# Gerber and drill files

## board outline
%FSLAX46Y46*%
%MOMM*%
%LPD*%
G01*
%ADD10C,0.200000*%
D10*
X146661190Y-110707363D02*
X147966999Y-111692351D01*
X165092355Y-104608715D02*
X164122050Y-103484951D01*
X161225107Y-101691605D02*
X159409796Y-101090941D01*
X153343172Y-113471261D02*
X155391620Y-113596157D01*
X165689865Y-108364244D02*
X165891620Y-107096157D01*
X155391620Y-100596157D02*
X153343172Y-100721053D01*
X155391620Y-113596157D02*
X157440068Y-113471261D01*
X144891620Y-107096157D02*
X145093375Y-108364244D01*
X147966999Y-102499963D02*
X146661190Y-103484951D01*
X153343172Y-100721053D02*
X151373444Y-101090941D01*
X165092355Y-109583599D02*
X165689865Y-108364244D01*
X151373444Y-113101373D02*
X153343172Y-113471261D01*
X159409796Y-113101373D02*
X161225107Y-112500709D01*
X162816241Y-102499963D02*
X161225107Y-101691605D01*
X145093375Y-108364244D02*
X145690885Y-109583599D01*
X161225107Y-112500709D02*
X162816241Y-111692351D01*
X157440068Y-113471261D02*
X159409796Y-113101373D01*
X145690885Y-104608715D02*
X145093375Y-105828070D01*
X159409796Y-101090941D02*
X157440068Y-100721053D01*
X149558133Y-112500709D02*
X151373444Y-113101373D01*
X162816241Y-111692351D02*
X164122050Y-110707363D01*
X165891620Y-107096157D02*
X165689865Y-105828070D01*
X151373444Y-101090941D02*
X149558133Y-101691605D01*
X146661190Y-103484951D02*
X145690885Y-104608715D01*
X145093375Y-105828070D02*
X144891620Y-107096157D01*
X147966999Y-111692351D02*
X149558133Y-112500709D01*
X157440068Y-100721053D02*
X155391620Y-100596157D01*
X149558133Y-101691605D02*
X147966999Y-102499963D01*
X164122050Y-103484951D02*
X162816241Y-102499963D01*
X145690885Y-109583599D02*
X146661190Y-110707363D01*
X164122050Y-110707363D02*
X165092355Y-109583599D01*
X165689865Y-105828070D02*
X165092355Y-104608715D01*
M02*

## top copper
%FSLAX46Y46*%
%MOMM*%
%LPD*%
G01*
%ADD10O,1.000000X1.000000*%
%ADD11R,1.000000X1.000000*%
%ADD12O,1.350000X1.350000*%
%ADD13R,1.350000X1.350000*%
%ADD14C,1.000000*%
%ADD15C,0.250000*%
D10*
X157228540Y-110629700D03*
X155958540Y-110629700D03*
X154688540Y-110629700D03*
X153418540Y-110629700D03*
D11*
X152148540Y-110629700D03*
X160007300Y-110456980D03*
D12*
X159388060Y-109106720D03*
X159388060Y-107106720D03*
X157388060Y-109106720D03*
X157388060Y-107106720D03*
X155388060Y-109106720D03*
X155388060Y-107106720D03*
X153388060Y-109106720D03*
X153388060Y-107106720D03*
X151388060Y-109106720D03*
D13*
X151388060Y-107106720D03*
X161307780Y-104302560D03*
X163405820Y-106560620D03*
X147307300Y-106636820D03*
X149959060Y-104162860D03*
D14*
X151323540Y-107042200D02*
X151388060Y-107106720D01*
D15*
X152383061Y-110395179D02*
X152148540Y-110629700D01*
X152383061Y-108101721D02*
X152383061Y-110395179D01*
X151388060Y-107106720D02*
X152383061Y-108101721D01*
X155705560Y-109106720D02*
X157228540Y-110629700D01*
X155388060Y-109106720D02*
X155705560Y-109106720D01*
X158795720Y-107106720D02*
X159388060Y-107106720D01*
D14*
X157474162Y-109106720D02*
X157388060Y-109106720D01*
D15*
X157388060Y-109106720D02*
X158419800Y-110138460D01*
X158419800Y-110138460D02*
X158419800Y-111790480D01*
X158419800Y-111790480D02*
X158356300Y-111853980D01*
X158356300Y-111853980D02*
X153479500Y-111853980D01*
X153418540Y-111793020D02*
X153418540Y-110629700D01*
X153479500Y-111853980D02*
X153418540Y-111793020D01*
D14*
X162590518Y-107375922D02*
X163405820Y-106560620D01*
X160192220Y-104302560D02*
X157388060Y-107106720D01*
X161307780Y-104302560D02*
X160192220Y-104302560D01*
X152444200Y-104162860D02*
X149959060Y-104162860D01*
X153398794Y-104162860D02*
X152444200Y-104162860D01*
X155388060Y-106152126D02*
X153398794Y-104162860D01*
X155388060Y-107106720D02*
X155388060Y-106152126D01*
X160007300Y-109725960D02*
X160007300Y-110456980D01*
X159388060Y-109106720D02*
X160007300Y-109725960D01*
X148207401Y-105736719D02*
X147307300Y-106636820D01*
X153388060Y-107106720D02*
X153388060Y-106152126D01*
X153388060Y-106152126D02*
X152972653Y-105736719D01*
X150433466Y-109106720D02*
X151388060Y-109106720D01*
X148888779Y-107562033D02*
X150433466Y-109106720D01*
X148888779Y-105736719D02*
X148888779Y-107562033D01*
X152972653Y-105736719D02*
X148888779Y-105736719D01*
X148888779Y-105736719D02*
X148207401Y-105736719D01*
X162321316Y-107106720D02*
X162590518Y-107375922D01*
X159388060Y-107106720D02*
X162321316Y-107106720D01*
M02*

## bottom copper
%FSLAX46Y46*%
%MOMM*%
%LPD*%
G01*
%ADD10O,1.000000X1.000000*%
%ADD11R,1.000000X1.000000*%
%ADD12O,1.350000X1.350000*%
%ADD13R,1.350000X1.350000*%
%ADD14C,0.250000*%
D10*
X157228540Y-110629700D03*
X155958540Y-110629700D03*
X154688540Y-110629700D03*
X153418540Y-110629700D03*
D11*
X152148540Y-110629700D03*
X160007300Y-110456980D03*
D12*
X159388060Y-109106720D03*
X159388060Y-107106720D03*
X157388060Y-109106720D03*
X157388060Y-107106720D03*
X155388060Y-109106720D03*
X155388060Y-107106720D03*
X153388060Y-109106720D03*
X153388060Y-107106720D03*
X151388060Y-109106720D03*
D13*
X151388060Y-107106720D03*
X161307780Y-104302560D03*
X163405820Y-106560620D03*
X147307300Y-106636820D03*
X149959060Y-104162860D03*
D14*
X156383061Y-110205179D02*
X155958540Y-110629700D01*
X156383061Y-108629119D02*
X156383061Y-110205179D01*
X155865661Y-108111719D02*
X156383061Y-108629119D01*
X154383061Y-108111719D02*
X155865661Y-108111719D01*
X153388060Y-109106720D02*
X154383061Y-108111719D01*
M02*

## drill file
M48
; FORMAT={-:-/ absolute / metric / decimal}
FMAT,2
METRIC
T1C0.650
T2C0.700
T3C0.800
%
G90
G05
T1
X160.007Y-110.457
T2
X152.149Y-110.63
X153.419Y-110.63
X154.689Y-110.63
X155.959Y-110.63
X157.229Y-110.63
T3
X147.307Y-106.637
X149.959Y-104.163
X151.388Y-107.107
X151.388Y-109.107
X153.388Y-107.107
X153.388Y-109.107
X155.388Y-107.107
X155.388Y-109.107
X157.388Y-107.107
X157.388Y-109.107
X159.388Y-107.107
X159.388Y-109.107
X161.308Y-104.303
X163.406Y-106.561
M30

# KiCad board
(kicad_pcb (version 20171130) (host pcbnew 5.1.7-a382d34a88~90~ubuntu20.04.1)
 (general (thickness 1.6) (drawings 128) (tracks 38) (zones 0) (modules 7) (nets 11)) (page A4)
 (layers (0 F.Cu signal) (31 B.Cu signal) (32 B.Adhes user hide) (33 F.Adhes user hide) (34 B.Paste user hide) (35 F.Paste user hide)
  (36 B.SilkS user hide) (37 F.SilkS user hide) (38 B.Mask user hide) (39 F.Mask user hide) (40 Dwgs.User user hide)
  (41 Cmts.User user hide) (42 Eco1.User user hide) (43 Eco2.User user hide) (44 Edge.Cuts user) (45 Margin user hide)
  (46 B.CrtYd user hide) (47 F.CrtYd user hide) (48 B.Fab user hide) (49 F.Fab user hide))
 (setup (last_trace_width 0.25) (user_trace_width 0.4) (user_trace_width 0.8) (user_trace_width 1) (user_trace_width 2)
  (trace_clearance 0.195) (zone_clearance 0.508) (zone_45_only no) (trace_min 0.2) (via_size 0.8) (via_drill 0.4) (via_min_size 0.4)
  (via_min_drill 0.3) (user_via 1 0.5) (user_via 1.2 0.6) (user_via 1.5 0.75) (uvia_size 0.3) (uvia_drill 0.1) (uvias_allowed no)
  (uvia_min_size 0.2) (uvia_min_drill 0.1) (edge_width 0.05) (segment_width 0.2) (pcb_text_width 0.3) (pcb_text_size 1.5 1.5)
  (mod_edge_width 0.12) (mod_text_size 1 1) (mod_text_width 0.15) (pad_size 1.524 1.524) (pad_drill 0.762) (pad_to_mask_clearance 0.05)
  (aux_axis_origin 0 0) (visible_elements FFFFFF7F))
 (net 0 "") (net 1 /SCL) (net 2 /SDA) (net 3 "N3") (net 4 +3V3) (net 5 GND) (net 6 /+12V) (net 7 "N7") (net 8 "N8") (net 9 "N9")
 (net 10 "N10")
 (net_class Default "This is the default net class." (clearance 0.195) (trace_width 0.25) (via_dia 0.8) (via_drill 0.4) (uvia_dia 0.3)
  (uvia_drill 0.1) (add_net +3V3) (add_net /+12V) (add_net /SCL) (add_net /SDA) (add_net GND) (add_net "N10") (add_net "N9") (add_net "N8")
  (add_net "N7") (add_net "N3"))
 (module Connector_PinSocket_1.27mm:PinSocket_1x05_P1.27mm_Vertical (layer F.Cu) (at 152.14854 110.6297 90)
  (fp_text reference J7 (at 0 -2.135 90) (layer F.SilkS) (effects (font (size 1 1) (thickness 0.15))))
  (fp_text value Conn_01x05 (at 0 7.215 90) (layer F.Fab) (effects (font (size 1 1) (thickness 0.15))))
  (pad 5 thru_hole oval (at 0 5.08 90) (size 1 1) (drill 0.7) (layers *.Cu *.Mask) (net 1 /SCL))
  (pad 4 thru_hole oval (at 0 3.81 90) (size 1 1) (drill 0.7) (layers *.Cu *.Mask) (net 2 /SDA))
  (pad 3 thru_hole oval (at 0 2.54 90) (size 1 1) (drill 0.7) (layers *.Cu *.Mask) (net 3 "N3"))
  (pad 2 thru_hole oval (at 0 1.27 90) (size 1 1) (drill 0.7) (layers *.Cu *.Mask) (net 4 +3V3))
  (pad 1 thru_hole rect (at 0 0 90) (size 1 1) (drill 0.7) (layers *.Cu *.Mask) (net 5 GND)))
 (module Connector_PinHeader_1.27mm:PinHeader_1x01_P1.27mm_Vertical (layer F.Cu) (at 160.0073 110.45698)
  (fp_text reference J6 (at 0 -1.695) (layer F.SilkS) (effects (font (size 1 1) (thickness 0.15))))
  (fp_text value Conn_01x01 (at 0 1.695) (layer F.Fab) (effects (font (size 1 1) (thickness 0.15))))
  (pad 1 thru_hole rect (at 0 0) (size 1 1) (drill 0.65) (layers *.Cu *.Mask) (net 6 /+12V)))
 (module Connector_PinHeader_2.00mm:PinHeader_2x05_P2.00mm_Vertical (layer B.Cu) (at 151.38806 107.10672 270)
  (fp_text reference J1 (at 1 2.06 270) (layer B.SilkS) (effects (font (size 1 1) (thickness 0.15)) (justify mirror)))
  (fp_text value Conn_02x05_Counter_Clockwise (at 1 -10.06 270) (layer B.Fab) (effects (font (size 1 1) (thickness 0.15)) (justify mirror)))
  (pad 10 thru_hole oval (at 2 -8 270) (size 1.35 1.35) (drill 0.8) (layers *.Cu *.Mask) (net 6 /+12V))
  (pad 9 thru_hole oval (at 0 -8 270) (size 1.35 1.35) (drill 0.8) (layers *.Cu *.Mask) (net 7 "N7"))
  (pad 8 thru_hole oval (at 2 -6 270) (size 1.35 1.35) (drill 0.8) (layers *.Cu *.Mask) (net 4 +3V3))
  (pad 7 thru_hole oval (at 0 -6 270) (size 1.35 1.35) (drill 0.8) (layers *.Cu *.Mask) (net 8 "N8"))
  (pad 6 thru_hole oval (at 2 -4 270) (size 1.35 1.35) (drill 0.8) (layers *.Cu *.Mask) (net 1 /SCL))
  (pad 5 thru_hole oval (at 0 -4 270) (size 1.35 1.35) (drill 0.8) (layers *.Cu *.Mask) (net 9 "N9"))
  (pad 4 thru_hole oval (at 2 -2 270) (size 1.35 1.35) (drill 0.8) (layers *.Cu *.Mask) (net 2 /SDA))
  (pad 3 thru_hole oval (at 0 -2 270) (size 1.35 1.35) (drill 0.8) (layers *.Cu *.Mask) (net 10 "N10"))
  (pad 2 thru_hole oval (at 2 0 270) (size 1.35 1.35) (drill 0.8) (layers *.Cu *.Mask) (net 10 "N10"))
  (pad 1 thru_hole rect (at 0 0 270) (size 1.35 1.35) (drill 0.8) (layers *.Cu *.Mask) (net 5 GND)))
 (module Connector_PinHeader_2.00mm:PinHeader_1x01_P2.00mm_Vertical (layer F.Cu) (at 161.30778 104.30256)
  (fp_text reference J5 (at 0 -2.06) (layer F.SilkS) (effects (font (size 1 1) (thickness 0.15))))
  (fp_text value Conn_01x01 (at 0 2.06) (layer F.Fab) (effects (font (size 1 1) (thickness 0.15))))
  (pad 1 thru_hole rect (at 0 0) (size 1.35 1.35) (drill 0.8) (layers *.Cu *.Mask) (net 8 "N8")))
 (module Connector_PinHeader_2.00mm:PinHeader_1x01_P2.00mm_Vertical (layer F.Cu) (at 163.40582 106.56062)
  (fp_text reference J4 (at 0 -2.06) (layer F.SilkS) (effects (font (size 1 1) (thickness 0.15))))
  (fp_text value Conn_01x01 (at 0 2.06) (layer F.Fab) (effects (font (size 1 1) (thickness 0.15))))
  (pad 1 thru_hole rect (at 0 0) (size 1.35 1.35) (drill 0.8) (layers *.Cu *.Mask) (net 7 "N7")))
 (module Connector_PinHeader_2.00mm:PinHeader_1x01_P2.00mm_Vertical (layer F.Cu) (at 147.3073 106.63682)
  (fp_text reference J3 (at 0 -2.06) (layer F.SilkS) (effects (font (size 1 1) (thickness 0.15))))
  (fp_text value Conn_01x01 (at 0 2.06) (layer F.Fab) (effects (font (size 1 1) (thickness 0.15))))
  (pad 1 thru_hole rect (at 0 0) (size 1.35 1.35) (drill 0.8) (layers *.Cu *.Mask) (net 10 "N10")))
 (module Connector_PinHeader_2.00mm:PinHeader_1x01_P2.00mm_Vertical (layer F.Cu) (at 149.95906 104.16286)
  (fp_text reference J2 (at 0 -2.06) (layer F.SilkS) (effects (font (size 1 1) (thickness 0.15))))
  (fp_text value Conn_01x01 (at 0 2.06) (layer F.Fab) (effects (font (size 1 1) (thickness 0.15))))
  (pad 1 thru_hole rect (at 0 0) (size 1.35 1.35) (drill 0.8) (layers *.Cu *.Mask) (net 9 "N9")))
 (gr_line (start 146.66119 110.707363) (end 147.966999 111.692351) (layer Edge.Cuts) (width 0.2))
 (gr_line (start 165.092355 104.608715) (end 164.12205 103.484951) (layer Edge.Cuts) (width 0.2))
 (gr_line (start 161.225107 101.691605) (end 159.409796 101.090941) (layer Edge.Cuts) (width 0.2))
 (gr_line (start 153.343172 113.471261) (end 155.39162 113.596157) (layer Edge.Cuts) (width 0.2))
 (gr_line (start 165.689865 108.364244) (end 165.89162 107.096157) (layer Edge.Cuts) (width 0.2))
 (gr_line (start 155.39162 100.596157) (end 153.343172 100.721053) (layer Edge.Cuts) (width 0.2))
 (gr_line (start 155.39162 113.596157) (end 157.440068 113.471261) (layer Edge.Cuts) (width 0.2))
 (gr_line (start 144.89162 107.096157) (end 145.093375 108.364244) (layer Edge.Cuts) (width 0.2))
 (gr_line (start 147.966999 102.499963) (end 146.66119 103.484951) (layer Edge.Cuts) (width 0.2))
 (gr_line (start 153.343172 100.721053) (end 151.373444 101.090941) (layer Edge.Cuts) (width 0.2))
 (gr_line (start 165.092355 109.583599) (end 165.689865 108.364244) (layer Edge.Cuts) (width 0.2))
 (gr_line (start 151.373444 113.101373) (end 153.343172 113.471261) (layer Edge.Cuts) (width 0.2))
 (gr_line (start 159.409796 113.101373) (end 161.225107 112.500709) (layer Edge.Cuts) (width 0.2))
 (gr_line (start 162.816241 102.499963) (end 161.225107 101.691605) (layer Edge.Cuts) (width 0.2))
 (gr_line (start 145.093375 108.364244) (end 145.690885 109.583599) (layer Edge.Cuts) (width 0.2))
 (gr_line (start 161.225107 112.500709) (end 162.816241 111.692351) (layer Edge.Cuts) (width 0.2))
 (gr_line (start 157.440068 113.471261) (end 159.409796 113.101373) (layer Edge.Cuts) (width 0.2))
 (gr_line (start 145.690885 104.608715) (end 145.093375 105.82807) (layer Edge.Cuts) (width 0.2))
 (gr_line (start 159.409796 101.090941) (end 157.440068 100.721053) (layer Edge.Cuts) (width 0.2))
 (gr_line (start 149.558133 112.500709) (end 151.373444 113.101373) (layer Edge.Cuts) (width 0.2))
 (gr_line (start 162.816241 111.692351) (end 164.12205 110.707363) (layer Edge.Cuts) (width 0.2))
 (gr_line (start 165.89162 107.096157) (end 165.689865 105.82807) (layer Edge.Cuts) (width 0.2))
 (gr_line (start 151.373444 101.090941) (end 149.558133 101.691605) (layer Edge.Cuts) (width 0.2))
 (gr_line (start 146.66119 103.484951) (end 145.690885 104.608715) (layer Edge.Cuts) (width 0.2))
 (gr_line (start 145.093375 105.82807) (end 144.89162 107.096157) (layer Edge.Cuts) (width 0.2))
 (gr_line (start 147.966999 111.692351) (end 149.558133 112.500709) (layer Edge.Cuts) (width 0.2))
 (gr_line (start 157.440068 100.721053) (end 155.39162 100.596157) (layer Edge.Cuts) (width 0.2))
 (gr_line (start 149.558133 101.691605) (end 147.966999 102.499963) (layer Edge.Cuts) (width 0.2))
 (gr_line (start 164.12205 103.484951) (end 162.816241 102.499963) (layer Edge.Cuts) (width 0.2))
 (gr_line (start 145.690885 109.583599) (end 146.66119 110.707363) (layer Edge.Cuts) (width 0.2))
 (gr_line (start 164.12205 110.707363) (end 165.092355 109.583599) (layer Edge.Cuts) (width 0.2))
 (gr_line (start 165.689865 105.82807) (end 165.092355 104.608715) (layer Edge.Cuts) (width 0.2))
 (segment (start 151.32354 107.0422) (end 151.38806 107.10672) (width 1) (layer F.Cu) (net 5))
 (segment (start 152.383061 110.395179) (end 152.14854 110.6297) (width 0.25) (layer F.Cu) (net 5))
 (segment (start 152.383061 108.101721) (end 152.383061 110.395179) (width 0.25) (layer F.Cu) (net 5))
 (segment (start 151.38806 107.10672) (end 152.383061 108.101721) (width 0.25) (layer F.Cu) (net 5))
 (segment (start 156.383061 110.205179) (end 155.95854 110.6297) (width 0.25) (layer B.Cu) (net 2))
 (segment (start 156.383061 108.629119) (end 156.383061 110.205179) (width 0.25) (layer B.Cu) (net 2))
 (segment (start 155.865661 108.111719) (end 156.383061 108.629119) (width 0.25) (layer B.Cu) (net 2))
 (segment (start 154.383061 108.111719) (end 155.865661 108.111719) (width 0.25) (layer B.Cu) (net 2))
 (segment (start 153.38806 109.10672) (end 154.383061 108.111719) (width 0.25) (layer B.Cu) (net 2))
 (segment (start 155.70556 109.10672) (end 157.22854 110.6297) (width 0.25) (layer F.Cu) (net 1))
 (segment (start 155.38806 109.10672) (end 155.70556 109.10672) (width 0.25) (layer F.Cu) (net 1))
 (segment (start 158.79572 107.10672) (end 159.38806 107.10672) (width 0.25) (layer F.Cu) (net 7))
 (segment (start 157.474162 109.10672) (end 157.38806 109.10672) (width 1) (layer F.Cu) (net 4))
 (segment (start 157.38806 109.10672) (end 158.4198 110.13846) (width 0.25) (layer F.Cu) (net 4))
 (segment (start 158.4198 110.13846) (end 158.4198 111.79048) (width 0.25) (layer F.Cu) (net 4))
 (segment (start 158.4198 111.79048) (end 158.3563 111.85398) (width 0.25) (layer F.Cu) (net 4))
 (segment (start 158.3563 111.85398) (end 153.4795 111.85398) (width 0.25) (layer F.Cu) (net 4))
 (segment (start 153.41854 111.79302) (end 153.41854 110.6297) (width 0.25) (layer F.Cu) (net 4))
 (segment (start 153.4795 111.85398) (end 153.41854 111.79302) (width 0.25) (layer F.Cu) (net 4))
 (segment (start 162.590518 107.375922) (end 163.40582 106.56062) (width 1) (layer F.Cu) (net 7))
 (segment (start 160.19222 104.30256) (end 157.38806 107.10672) (width 1) (layer F.Cu) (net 8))
 (segment (start 161.30778 104.30256) (end 160.19222 104.30256) (width 1) (layer F.Cu) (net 8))
 (segment (start 152.4442 104.16286) (end 149.95906 104.16286) (width 1) (layer F.Cu) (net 9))
 (segment (start 153.398794 104.16286) (end 152.4442 104.16286) (width 1) (layer F.Cu) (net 9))
 (segment (start 155.38806 106.152126) (end 153.398794 104.16286) (width 1) (layer F.Cu) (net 9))
 (segment (start 155.38806 107.10672) (end 155.38806 106.152126) (width 1) (layer F.Cu) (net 9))
 (segment (start 160.0073 109.72596) (end 160.0073 110.45698) (width 1) (layer F.Cu) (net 6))
 (segment (start 159.38806 109.10672) (end 160.0073 109.72596) (width 1) (layer F.Cu) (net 6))
 (segment (start 148.207401 105.736719) (end 147.3073 106.63682) (width 1) (layer F.Cu) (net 10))
 (segment (start 153.38806 107.10672) (end 153.38806 106.152126) (width 1) (layer F.Cu) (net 10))
 (segment (start 153.38806 106.152126) (end 152.972653 105.736719) (width 1) (layer F.Cu) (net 10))
 (segment (start 150.433466 109.10672) (end 151.38806 109.10672) (width 1) (layer F.Cu) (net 10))
 (segment (start 148.888779 107.562033) (end 150.433466 109.10672) (width 1) (layer F.Cu) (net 10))
 (segment (start 148.888779 105.736719) (end 148.888779 107.562033) (width 1) (layer F.Cu) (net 10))
 (segment (start 152.972653 105.736719) (end 148.888779 105.736719) (width 1) (layer F.Cu) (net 10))
 (segment (start 148.888779 105.736719) (end 148.207401 105.736719) (width 1) (layer F.Cu) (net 10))
 (segment (start 162.321316 107.10672) (end 162.590518 107.375922) (width 1) (layer F.Cu) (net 7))
 (segment (start 159.38806 107.10672) (end 162.321316 107.10672) (width 1) (layer F.Cu) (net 7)))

